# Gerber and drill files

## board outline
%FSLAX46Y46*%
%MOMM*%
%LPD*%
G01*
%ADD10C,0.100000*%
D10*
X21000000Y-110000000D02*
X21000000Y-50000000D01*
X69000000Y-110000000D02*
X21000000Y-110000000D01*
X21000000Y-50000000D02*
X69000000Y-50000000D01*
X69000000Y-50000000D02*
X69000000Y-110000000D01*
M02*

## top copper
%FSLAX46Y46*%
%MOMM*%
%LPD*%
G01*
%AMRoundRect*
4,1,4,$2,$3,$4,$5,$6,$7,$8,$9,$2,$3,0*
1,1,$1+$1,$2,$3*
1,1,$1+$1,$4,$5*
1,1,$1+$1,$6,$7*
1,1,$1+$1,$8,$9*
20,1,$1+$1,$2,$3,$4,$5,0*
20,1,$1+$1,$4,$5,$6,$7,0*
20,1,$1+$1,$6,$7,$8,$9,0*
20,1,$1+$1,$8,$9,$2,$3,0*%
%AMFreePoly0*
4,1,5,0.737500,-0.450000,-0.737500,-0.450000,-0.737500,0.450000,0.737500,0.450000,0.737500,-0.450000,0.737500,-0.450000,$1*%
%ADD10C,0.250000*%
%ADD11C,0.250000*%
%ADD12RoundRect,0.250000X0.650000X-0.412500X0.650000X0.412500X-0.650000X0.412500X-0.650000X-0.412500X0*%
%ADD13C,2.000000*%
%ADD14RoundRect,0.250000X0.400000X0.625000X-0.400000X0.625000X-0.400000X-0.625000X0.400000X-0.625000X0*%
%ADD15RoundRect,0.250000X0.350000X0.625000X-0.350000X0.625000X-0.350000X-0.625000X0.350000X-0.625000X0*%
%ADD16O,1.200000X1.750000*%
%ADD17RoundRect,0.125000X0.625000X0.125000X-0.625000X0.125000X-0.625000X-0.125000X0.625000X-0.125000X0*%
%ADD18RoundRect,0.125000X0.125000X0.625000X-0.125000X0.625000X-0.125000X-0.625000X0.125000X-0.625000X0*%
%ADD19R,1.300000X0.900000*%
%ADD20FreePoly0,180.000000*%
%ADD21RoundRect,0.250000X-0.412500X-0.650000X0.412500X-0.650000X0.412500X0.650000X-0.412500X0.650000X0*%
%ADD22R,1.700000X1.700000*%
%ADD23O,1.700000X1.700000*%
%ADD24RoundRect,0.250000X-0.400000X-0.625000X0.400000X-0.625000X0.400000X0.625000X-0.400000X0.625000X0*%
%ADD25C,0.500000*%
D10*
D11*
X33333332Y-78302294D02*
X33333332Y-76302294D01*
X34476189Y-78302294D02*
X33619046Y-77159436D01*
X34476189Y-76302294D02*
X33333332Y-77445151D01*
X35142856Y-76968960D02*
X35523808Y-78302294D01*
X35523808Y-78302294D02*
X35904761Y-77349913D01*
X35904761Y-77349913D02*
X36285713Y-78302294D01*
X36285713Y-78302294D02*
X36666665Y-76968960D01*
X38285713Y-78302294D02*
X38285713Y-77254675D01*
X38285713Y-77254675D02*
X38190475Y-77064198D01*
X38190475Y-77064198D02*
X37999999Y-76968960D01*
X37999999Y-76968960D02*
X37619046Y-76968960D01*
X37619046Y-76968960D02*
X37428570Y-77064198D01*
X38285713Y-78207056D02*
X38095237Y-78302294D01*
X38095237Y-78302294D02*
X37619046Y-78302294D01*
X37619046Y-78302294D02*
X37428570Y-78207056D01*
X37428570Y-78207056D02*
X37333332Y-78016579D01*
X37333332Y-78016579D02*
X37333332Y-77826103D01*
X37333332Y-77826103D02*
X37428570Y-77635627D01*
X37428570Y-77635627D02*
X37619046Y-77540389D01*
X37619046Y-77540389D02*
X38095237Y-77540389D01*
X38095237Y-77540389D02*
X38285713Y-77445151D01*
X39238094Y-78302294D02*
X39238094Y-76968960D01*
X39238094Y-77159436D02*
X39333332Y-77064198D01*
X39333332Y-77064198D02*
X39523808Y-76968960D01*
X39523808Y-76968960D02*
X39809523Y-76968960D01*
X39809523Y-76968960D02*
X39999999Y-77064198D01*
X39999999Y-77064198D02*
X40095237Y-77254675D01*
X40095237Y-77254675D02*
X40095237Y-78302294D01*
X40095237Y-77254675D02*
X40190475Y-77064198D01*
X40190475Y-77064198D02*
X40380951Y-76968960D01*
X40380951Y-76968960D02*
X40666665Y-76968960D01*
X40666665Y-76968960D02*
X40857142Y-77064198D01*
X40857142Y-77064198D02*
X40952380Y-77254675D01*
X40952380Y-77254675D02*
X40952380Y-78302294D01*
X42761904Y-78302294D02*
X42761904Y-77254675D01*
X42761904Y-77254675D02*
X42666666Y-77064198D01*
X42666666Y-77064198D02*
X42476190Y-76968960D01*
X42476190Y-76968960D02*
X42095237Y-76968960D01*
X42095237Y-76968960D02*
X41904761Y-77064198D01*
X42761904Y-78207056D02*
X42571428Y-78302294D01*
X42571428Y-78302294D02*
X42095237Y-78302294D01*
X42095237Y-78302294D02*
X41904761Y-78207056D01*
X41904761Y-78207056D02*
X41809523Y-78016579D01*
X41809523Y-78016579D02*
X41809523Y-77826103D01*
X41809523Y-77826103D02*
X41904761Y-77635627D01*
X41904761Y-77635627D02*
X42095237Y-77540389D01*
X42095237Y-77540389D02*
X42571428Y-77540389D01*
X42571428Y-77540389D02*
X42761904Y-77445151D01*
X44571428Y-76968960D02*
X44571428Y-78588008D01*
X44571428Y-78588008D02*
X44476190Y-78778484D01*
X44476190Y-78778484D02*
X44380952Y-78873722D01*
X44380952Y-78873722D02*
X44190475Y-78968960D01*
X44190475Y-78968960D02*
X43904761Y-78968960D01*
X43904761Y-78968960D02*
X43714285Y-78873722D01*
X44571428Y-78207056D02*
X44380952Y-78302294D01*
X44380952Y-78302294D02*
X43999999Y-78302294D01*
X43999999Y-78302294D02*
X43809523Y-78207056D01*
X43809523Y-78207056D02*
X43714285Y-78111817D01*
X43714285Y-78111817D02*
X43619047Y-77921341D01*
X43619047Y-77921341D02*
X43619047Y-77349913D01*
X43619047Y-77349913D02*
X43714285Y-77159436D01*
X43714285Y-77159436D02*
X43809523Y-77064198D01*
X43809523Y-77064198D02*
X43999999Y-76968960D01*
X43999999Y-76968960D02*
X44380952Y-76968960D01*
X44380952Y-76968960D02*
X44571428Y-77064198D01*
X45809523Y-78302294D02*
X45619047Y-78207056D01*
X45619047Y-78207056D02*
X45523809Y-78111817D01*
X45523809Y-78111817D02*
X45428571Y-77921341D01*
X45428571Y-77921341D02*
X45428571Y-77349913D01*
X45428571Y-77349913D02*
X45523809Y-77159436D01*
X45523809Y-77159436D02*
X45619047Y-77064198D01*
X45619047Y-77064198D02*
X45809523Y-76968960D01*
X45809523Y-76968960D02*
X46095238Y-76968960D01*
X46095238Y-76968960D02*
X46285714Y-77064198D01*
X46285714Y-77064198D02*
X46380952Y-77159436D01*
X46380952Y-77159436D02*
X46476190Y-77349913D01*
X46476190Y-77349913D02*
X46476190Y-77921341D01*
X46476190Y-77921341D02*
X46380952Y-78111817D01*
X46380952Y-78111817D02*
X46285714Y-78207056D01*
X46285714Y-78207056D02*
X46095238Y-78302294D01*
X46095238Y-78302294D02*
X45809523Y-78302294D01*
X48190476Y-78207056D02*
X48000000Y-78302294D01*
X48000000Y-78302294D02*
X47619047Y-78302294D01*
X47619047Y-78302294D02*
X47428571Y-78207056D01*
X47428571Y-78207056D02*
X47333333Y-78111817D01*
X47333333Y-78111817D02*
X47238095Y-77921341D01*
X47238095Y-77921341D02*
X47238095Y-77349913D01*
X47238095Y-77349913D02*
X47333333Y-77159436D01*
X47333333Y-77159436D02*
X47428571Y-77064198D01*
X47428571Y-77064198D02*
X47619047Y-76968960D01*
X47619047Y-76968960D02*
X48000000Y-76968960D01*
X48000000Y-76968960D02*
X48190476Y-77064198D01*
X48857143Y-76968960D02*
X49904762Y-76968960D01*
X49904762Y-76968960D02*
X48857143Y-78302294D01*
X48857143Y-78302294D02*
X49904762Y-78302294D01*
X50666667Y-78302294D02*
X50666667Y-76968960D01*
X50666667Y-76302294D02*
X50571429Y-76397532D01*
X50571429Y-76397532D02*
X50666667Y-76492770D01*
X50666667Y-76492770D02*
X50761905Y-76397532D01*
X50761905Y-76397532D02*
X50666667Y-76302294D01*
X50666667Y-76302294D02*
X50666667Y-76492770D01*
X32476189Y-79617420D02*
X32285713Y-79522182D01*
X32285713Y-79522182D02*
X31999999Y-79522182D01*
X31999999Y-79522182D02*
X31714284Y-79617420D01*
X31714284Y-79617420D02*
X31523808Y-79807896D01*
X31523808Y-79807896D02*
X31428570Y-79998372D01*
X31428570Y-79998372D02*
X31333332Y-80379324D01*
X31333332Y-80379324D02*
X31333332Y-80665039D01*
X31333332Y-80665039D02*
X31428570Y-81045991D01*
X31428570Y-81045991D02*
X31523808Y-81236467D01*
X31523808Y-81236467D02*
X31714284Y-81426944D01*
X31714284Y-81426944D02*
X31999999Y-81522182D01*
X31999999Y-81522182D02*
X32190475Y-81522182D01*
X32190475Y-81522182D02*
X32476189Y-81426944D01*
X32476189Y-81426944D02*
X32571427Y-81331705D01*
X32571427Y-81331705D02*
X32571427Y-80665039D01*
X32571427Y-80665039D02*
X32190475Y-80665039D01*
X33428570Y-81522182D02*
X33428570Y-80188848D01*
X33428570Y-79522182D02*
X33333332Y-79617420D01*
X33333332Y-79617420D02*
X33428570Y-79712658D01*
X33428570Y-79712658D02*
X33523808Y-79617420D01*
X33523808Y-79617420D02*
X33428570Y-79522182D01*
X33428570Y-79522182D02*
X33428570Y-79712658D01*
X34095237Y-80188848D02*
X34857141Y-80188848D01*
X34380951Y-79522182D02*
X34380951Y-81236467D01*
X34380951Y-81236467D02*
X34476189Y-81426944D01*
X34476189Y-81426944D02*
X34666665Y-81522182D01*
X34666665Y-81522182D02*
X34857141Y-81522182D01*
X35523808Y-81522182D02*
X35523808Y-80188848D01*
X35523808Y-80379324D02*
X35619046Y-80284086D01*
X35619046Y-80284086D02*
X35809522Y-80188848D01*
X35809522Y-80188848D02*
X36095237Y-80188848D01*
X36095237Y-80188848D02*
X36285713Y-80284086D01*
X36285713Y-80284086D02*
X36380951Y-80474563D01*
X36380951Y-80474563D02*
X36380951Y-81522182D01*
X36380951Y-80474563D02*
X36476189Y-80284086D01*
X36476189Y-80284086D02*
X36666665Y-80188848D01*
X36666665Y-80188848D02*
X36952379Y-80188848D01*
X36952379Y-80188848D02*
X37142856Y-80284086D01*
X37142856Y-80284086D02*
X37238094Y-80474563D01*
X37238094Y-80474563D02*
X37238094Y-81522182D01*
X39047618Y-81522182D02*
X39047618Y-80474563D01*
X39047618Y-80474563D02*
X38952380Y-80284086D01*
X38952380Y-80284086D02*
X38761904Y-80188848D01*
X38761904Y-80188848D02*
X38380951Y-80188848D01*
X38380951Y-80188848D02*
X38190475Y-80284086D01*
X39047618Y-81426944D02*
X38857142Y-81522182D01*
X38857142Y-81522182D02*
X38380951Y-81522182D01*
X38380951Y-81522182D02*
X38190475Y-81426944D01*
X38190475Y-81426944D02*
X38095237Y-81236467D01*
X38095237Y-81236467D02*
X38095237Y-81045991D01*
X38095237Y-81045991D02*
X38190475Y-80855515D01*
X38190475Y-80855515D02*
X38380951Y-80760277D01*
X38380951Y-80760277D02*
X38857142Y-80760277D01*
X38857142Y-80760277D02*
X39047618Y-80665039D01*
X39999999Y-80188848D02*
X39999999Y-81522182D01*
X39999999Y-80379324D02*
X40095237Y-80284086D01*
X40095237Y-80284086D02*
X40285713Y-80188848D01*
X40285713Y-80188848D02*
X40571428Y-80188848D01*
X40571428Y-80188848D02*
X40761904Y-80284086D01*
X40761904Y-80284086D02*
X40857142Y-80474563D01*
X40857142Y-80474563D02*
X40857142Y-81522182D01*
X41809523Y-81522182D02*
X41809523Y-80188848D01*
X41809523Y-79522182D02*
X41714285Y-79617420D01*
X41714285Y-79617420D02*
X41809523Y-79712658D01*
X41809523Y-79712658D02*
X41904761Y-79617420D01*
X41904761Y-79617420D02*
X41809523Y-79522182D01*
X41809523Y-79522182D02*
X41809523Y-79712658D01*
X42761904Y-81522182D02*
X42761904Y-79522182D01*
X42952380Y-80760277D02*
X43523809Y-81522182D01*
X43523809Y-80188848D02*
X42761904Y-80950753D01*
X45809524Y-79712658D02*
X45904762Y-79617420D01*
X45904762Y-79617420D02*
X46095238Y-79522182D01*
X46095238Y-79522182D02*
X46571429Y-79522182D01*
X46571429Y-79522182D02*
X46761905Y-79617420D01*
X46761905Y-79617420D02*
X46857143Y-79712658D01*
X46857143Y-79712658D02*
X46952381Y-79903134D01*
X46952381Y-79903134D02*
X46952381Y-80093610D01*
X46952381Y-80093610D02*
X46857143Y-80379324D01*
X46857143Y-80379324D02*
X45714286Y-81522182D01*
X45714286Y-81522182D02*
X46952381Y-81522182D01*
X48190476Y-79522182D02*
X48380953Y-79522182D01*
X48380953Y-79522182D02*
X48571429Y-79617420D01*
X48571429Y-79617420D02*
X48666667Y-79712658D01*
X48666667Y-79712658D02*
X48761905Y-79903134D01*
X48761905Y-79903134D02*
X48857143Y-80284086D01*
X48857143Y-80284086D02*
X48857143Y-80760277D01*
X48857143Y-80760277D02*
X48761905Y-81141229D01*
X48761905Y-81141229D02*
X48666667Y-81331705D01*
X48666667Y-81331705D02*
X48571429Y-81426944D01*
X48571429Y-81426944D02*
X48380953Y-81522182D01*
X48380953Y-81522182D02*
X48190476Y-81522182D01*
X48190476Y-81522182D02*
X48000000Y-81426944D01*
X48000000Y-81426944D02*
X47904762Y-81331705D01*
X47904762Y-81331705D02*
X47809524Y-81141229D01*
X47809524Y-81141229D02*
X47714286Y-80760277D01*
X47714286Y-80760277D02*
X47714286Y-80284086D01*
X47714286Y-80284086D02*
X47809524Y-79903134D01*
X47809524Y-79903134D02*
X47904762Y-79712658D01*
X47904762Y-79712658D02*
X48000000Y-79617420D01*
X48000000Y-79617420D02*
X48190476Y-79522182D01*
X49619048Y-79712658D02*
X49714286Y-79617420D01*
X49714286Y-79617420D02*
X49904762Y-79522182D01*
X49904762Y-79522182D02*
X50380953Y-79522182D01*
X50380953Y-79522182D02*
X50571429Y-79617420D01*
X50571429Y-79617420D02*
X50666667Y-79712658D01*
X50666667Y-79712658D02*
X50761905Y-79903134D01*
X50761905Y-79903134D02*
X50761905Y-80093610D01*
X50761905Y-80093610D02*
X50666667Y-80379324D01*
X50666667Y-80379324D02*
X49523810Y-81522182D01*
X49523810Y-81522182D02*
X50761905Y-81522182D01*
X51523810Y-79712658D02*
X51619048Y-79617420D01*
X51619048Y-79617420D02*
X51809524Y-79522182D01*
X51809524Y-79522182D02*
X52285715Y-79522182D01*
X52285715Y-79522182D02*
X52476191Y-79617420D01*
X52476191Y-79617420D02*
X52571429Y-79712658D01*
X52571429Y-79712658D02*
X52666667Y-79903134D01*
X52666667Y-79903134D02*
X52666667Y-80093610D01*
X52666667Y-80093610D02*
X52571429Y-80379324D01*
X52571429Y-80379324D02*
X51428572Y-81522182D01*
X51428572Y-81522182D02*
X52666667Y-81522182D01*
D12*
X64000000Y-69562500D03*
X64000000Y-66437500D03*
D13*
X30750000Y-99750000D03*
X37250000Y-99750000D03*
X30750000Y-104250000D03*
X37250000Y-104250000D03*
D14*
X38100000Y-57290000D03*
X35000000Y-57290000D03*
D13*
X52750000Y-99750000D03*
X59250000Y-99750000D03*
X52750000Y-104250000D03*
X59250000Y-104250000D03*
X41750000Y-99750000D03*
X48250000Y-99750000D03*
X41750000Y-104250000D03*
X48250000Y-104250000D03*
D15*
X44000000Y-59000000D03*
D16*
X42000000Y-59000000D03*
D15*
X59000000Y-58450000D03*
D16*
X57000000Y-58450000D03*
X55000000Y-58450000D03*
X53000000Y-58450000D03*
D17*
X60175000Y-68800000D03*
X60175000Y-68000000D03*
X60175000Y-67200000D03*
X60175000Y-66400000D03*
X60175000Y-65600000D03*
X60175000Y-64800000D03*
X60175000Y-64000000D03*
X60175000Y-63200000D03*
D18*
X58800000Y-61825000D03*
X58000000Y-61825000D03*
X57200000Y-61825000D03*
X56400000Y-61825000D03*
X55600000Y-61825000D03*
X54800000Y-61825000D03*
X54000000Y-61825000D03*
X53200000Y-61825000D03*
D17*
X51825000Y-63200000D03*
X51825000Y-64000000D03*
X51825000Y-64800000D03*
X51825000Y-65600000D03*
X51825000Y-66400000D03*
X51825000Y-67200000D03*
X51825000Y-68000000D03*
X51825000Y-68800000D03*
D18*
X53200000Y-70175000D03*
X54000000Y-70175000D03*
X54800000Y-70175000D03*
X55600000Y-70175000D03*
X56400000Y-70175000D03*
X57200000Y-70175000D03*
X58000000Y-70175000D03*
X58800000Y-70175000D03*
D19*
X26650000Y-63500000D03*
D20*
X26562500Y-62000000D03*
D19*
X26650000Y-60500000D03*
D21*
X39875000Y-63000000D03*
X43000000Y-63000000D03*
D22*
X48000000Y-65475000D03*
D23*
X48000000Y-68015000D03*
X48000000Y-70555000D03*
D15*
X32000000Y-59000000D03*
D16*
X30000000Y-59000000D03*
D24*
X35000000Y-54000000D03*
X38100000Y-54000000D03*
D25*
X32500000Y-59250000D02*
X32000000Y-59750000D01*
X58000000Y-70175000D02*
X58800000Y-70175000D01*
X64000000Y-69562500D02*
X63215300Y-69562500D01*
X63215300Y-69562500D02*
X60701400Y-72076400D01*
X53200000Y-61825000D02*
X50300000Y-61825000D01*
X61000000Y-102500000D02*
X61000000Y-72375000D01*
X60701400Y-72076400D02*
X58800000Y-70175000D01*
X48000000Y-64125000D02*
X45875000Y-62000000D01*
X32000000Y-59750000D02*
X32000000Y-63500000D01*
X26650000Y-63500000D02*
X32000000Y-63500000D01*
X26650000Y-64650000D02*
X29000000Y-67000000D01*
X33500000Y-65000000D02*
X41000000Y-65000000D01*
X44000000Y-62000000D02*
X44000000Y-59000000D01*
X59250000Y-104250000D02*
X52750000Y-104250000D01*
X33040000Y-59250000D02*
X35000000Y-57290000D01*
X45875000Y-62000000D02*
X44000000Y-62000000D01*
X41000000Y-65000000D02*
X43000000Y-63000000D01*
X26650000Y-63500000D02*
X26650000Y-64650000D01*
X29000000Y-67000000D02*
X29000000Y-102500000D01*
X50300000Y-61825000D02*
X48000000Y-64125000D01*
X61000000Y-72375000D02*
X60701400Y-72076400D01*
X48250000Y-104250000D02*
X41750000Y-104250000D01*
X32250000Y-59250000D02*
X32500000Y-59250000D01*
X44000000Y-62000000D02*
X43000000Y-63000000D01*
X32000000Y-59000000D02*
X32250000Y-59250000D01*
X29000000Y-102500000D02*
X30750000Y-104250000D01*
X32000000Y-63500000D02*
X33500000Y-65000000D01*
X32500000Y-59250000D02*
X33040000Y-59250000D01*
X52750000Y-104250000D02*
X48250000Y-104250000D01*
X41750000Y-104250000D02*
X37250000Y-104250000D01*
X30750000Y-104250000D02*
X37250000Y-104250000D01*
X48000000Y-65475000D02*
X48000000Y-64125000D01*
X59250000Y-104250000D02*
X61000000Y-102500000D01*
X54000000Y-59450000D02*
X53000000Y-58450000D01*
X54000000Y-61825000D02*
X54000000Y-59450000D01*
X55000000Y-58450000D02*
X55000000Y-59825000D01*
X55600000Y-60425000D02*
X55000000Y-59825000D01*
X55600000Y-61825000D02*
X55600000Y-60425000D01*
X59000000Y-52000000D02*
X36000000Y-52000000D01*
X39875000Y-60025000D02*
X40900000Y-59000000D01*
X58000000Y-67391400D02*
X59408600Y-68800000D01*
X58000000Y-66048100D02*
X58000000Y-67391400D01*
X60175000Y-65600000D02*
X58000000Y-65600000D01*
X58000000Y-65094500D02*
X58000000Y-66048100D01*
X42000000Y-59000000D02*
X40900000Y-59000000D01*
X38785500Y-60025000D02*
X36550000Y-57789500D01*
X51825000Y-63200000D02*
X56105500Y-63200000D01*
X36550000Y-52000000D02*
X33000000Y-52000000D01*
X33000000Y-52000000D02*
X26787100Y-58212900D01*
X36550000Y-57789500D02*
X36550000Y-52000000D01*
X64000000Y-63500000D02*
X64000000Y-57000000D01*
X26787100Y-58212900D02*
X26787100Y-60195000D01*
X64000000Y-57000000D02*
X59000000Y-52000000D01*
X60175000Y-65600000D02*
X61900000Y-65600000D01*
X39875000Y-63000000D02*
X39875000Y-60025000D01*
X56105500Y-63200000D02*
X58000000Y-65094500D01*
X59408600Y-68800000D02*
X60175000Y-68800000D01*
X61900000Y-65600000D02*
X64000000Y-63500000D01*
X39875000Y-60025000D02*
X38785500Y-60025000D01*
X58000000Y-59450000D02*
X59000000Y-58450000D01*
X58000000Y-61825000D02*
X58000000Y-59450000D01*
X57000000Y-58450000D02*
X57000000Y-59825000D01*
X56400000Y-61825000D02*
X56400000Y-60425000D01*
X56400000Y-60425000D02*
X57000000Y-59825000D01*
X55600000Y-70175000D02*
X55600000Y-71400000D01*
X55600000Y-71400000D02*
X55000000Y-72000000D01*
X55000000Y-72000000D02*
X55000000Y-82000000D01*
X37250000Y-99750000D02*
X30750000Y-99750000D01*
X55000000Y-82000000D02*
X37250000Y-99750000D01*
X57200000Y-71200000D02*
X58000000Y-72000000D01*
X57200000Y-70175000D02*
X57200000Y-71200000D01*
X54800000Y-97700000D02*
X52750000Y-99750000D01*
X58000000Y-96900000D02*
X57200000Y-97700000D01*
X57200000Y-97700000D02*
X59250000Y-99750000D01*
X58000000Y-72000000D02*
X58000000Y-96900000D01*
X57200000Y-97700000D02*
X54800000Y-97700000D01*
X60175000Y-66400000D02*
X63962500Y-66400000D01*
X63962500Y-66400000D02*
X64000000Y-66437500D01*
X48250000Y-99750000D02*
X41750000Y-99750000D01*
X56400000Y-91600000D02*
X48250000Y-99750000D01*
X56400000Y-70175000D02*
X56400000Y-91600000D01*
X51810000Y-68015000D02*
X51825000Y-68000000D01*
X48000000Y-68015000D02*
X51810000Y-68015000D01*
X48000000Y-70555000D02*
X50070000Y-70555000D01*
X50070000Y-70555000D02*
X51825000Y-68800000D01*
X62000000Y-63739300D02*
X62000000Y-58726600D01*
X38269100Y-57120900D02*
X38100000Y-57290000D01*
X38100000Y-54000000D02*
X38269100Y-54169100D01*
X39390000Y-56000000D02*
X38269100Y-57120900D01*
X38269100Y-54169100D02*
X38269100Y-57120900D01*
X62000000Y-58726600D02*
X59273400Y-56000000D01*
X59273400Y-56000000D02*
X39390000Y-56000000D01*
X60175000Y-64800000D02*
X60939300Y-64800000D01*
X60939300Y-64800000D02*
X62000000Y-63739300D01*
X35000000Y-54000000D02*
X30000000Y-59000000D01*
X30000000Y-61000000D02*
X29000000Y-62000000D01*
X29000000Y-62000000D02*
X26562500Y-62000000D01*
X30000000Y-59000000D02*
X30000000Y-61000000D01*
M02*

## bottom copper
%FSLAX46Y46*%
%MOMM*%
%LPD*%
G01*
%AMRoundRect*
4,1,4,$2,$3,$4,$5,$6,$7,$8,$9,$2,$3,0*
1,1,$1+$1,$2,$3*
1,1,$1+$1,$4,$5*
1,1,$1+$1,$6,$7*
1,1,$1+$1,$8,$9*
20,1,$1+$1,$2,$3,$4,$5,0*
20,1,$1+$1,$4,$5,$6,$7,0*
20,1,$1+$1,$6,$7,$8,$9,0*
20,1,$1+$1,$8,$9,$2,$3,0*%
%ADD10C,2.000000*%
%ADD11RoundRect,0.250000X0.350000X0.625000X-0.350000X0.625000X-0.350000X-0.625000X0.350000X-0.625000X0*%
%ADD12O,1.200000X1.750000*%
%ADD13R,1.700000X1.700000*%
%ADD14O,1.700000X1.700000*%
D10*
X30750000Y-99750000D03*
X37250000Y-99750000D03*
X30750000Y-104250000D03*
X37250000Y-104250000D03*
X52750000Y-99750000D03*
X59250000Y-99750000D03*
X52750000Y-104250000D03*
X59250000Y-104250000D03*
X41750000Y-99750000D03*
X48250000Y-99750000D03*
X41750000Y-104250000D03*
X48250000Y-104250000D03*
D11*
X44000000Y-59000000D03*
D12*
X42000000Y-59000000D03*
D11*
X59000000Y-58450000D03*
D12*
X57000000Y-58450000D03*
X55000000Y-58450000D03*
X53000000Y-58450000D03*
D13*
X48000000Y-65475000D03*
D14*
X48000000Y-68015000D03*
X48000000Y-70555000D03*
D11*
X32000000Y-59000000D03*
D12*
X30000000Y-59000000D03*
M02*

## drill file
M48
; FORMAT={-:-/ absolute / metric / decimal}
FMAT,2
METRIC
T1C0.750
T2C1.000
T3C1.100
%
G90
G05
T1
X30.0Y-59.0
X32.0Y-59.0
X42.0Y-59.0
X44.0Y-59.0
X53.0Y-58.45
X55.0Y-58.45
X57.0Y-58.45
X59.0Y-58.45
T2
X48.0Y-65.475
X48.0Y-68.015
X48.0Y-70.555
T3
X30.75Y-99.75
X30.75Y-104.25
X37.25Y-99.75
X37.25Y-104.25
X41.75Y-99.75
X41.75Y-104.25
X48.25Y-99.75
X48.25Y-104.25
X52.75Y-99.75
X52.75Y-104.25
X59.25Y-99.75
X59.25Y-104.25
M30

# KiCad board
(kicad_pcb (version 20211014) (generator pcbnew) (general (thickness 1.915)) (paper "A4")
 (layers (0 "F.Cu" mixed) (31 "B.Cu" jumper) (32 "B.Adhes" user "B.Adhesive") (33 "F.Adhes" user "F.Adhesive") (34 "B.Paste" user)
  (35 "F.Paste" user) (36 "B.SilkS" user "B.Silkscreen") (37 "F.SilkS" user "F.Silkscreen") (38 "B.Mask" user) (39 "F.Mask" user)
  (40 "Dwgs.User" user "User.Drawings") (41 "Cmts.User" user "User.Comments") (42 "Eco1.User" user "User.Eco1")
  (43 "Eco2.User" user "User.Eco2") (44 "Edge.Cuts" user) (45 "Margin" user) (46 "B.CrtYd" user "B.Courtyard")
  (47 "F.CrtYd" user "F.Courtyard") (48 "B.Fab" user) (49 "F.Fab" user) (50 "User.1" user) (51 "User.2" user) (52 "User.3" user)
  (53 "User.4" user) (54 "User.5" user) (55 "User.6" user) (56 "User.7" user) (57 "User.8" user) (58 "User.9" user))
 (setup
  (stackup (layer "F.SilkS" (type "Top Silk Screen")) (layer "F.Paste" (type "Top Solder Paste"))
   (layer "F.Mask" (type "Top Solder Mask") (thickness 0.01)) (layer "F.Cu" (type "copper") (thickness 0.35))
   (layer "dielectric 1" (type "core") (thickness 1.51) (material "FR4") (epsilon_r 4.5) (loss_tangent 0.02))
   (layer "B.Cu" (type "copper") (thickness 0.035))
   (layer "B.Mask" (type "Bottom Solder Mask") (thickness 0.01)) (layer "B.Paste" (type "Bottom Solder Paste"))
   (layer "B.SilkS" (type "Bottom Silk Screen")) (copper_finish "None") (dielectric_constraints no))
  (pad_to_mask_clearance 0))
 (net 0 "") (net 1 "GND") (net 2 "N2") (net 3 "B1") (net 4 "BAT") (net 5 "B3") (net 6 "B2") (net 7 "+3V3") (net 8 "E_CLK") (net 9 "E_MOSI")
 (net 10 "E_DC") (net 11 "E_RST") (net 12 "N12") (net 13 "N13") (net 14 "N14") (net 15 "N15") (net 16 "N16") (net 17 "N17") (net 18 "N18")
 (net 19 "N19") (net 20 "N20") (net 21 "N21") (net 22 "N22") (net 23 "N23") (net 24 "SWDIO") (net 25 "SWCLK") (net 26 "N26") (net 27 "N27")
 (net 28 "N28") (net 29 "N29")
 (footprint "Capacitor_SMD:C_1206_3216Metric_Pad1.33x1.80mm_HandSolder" (layer "F.Cu") (at 64 68 90)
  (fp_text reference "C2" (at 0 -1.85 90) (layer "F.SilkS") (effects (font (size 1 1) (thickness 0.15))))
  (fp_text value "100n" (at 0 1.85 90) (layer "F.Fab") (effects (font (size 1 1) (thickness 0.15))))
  (pad "1" smd roundrect (at -1.5625 0 90) (size 1.325 1.8) (layers "F.Cu" "F.Paste" "F.Mask") (roundrect_rratio 0.188679) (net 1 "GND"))
  (pad "2" smd roundrect (at 1.5625 0 90) (size 1.325 1.8) (layers "F.Cu" "F.Paste" "F.Mask") (roundrect_rratio 0.188679) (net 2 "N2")))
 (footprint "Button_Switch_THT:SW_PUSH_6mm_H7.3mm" (layer "F.Cu") (at 30.75 99.75)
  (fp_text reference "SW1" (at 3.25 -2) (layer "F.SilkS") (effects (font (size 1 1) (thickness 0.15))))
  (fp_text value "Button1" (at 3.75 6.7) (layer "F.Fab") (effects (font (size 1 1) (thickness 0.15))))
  (pad "1" thru_hole circle (at 0 0 90) (size 2 2) (drill 1.1) (layers *.Cu *.Mask) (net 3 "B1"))
  (pad "1" thru_hole circle (at 6.5 0 90) (size 2 2) (drill 1.1) (layers *.Cu *.Mask) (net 3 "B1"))
  (pad "2" thru_hole circle (at 0 4.5 90) (size 2 2) (drill 1.1) (layers *.Cu *.Mask) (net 1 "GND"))
  (pad "2" thru_hole circle (at 6.5 4.5 90) (size 2 2) (drill 1.1) (layers *.Cu *.Mask) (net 1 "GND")))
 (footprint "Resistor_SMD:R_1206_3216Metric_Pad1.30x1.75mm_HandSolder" (layer "F.Cu") (at 36.55 57.29 180)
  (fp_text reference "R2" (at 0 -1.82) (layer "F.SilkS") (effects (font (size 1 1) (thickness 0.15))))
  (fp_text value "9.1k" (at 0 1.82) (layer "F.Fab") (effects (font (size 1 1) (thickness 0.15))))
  (pad "1" smd roundrect (at -1.55 0 180) (size 1.3 1.75) (layers "F.Cu" "F.Paste" "F.Mask") (roundrect_rratio 0.192308) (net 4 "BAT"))
  (pad "2" smd roundrect (at 1.55 0 180) (size 1.3 1.75) (layers "F.Cu" "F.Paste" "F.Mask") (roundrect_rratio 0.192308) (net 1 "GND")))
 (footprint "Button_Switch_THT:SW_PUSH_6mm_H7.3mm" (layer "F.Cu") (at 52.75 99.75)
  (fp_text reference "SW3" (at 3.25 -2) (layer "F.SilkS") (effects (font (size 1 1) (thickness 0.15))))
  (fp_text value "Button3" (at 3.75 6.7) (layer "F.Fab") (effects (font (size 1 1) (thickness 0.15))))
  (pad "1" thru_hole circle (at 0 0 90) (size 2 2) (drill 1.1) (layers *.Cu *.Mask) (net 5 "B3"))
  (pad "1" thru_hole circle (at 6.5 0 90) (size 2 2) (drill 1.1) (layers *.Cu *.Mask) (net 5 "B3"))
  (pad "2" thru_hole circle (at 0 4.5 90) (size 2 2) (drill 1.1) (layers *.Cu *.Mask) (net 1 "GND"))
  (pad "2" thru_hole circle (at 6.5 4.5 90) (size 2 2) (drill 1.1) (layers *.Cu *.Mask) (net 1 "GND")))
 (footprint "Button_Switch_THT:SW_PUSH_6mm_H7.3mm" (layer "F.Cu") (at 41.75 99.75)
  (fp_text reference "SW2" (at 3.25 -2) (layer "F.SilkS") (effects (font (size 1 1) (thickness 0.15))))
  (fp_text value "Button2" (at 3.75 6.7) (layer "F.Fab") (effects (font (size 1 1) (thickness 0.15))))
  (pad "1" thru_hole circle (at 0 0 90) (size 2 2) (drill 1.1) (layers *.Cu *.Mask) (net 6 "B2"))
  (pad "1" thru_hole circle (at 6.5 0 90) (size 2 2) (drill 1.1) (layers *.Cu *.Mask) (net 6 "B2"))
  (pad "2" thru_hole circle (at 0 4.5 90) (size 2 2) (drill 1.1) (layers *.Cu *.Mask) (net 1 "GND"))
  (pad "2" thru_hole circle (at 6.5 4.5 90) (size 2 2) (drill 1.1) (layers *.Cu *.Mask) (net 1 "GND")))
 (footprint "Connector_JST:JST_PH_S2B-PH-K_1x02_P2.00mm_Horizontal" (layer "F.Cu") (at 44 59 180)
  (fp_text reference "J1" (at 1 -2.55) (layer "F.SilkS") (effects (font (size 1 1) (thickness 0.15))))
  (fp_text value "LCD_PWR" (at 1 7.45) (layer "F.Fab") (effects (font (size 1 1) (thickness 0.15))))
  (pad "1" thru_hole roundrect (at 0 0 180) (size 1.2 1.75) (drill 0.75) (layers *.Cu *.Mask) (roundrect_rratio 0.208333) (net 1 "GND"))
  (pad "2" thru_hole oval (at 2 0 180) (size 1.2 1.75) (drill 0.75) (layers *.Cu *.Mask) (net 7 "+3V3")))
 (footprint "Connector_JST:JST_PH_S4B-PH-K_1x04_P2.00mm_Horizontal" (layer "F.Cu") (at 59 58.45 180)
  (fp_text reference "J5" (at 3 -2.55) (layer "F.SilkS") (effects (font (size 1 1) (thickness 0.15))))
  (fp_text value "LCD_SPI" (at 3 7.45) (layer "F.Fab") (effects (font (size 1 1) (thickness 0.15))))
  (pad "1" thru_hole roundrect (at 0 0 180) (size 1.2 1.75) (drill 0.75) (layers *.Cu *.Mask) (roundrect_rratio 0.208333) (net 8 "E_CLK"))
  (pad "2" thru_hole oval (at 2 0 180) (size 1.2 1.75) (drill 0.75) (layers *.Cu *.Mask) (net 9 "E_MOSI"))
  (pad "3" thru_hole oval (at 4 0 180) (size 1.2 1.75) (drill 0.75) (layers *.Cu *.Mask) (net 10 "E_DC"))
  (pad "4" thru_hole oval (at 6 0 180) (size 1.2 1.75) (drill 0.75) (layers *.Cu *.Mask) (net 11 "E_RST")))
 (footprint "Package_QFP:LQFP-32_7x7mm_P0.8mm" (layer "F.Cu") (at 56 66 180)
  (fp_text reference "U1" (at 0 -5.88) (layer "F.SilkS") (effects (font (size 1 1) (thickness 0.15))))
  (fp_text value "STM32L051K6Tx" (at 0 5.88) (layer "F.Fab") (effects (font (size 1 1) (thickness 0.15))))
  (pad "1" smd roundrect (at -4.175 -2.8 180) (size 1.5 0.5) (layers "F.Cu" "F.Paste" "F.Mask") (roundrect_rratio 0.25) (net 7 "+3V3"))
  (pad "2" smd roundrect (at -4.175 -2 180) (size 1.5 0.5) (layers "F.Cu" "F.Paste" "F.Mask") (roundrect_rratio 0.25) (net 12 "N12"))
  (pad "3" smd roundrect (at -4.175 -1.2 180) (size 1.5 0.5) (layers "F.Cu" "F.Paste" "F.Mask") (roundrect_rratio 0.25) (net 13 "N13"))
  (pad "4" smd roundrect (at -4.175 -0.4 180) (size 1.5 0.5) (layers "F.Cu" "F.Paste" "F.Mask") (roundrect_rratio 0.25) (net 2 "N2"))
  (pad "5" smd roundrect (at -4.175 0.4 180) (size 1.5 0.5) (layers "F.Cu" "F.Paste" "F.Mask") (roundrect_rratio 0.25) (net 7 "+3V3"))
  (pad "6" smd roundrect (at -4.175 1.2 180) (size 1.5 0.5) (layers "F.Cu" "F.Paste" "F.Mask") (roundrect_rratio 0.25) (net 4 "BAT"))
  (pad "7" smd roundrect (at -4.175 2 180) (size 1.5 0.5) (layers "F.Cu" "F.Paste" "F.Mask") (roundrect_rratio 0.25) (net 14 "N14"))
  (pad "8" smd roundrect (at -4.175 2.8 180) (size 1.5 0.5) (layers "F.Cu" "F.Paste" "F.Mask") (roundrect_rratio 0.25) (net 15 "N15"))
  (pad "9" smd roundrect (at -2.8 4.175 180) (size 0.5 1.5) (layers "F.Cu" "F.Paste" "F.Mask") (roundrect_rratio 0.25) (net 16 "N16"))
  (pad "10" smd roundrect (at -2 4.175 180) (size 0.5 1.5) (layers "F.Cu" "F.Paste" "F.Mask") (roundrect_rratio 0.25) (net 8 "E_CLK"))
  (pad "11" smd roundrect (at -1.2 4.175 180) (size 0.5 1.5) (layers "F.Cu" "F.Paste" "F.Mask") (roundrect_rratio 0.25) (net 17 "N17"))
  (pad "12" smd roundrect (at -0.4 4.175 180) (size 0.5 1.5) (layers "F.Cu" "F.Paste" "F.Mask") (roundrect_rratio 0.25) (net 9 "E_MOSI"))
  (pad "13" smd roundrect (at 0.4 4.175 180) (size 0.5 1.5) (layers "F.Cu" "F.Paste" "F.Mask") (roundrect_rratio 0.25) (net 10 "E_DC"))
  (pad "14" smd roundrect (at 1.2 4.175 180) (size 0.5 1.5) (layers "F.Cu" "F.Paste" "F.Mask") (roundrect_rratio 0.25) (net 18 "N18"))
  (pad "15" smd roundrect (at 2 4.175 180) (size 0.5 1.5) (layers "F.Cu" "F.Paste" "F.Mask") (roundrect_rratio 0.25) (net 11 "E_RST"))
  (pad "16" smd roundrect (at 2.8 4.175 180) (size 0.5 1.5) (layers "F.Cu" "F.Paste" "F.Mask") (roundrect_rratio 0.25) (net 1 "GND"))
  (pad "17" smd roundrect (at 4.175 2.8 180) (size 1.5 0.5) (layers "F.Cu" "F.Paste" "F.Mask") (roundrect_rratio 0.25) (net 7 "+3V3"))
  (pad "18" smd roundrect (at 4.175 2 180) (size 1.5 0.5) (layers "F.Cu" "F.Paste" "F.Mask") (roundrect_rratio 0.25) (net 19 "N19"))
  (pad "19" smd roundrect (at 4.175 1.2 180) (size 1.5 0.5) (layers "F.Cu" "F.Paste" "F.Mask") (roundrect_rratio 0.25) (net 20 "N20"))
  (pad "20" smd roundrect (at 4.175 0.4 180) (size 1.5 0.5) (layers "F.Cu" "F.Paste" "F.Mask") (roundrect_rratio 0.25) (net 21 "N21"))
  (pad "21" smd roundrect (at 4.175 -0.4 180) (size 1.5 0.5) (layers "F.Cu" "F.Paste" "F.Mask") (roundrect_rratio 0.25) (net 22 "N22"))
  (pad "22" smd roundrect (at 4.175 -1.2 180) (size 1.5 0.5) (layers "F.Cu" "F.Paste" "F.Mask") (roundrect_rratio 0.25) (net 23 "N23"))
  (pad "23" smd roundrect (at 4.175 -2 180) (size 1.5 0.5) (layers "F.Cu" "F.Paste" "F.Mask") (roundrect_rratio 0.25) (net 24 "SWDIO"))
  (pad "24" smd roundrect (at 4.175 -2.8 180) (size 1.5 0.5) (layers "F.Cu" "F.Paste" "F.Mask") (roundrect_rratio 0.25) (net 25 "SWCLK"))
  (pad "25" smd roundrect (at 2.8 -4.175 180) (size 0.5 1.5) (layers "F.Cu" "F.Paste" "F.Mask") (roundrect_rratio 0.25) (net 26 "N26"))
  (pad "26" smd roundrect (at 2 -4.175 180) (size 0.5 1.5) (layers "F.Cu" "F.Paste" "F.Mask") (roundrect_rratio 0.25) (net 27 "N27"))
  (pad "27" smd roundrect (at 1.2 -4.175 180) (size 0.5 1.5) (layers "F.Cu" "F.Paste" "F.Mask") (roundrect_rratio 0.25) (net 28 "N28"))
  (pad "28" smd roundrect (at 0.4 -4.175 180) (size 0.5 1.5) (layers "F.Cu" "F.Paste" "F.Mask") (roundrect_rratio 0.25) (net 3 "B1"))
  (pad "29" smd roundrect (at -0.4 -4.175 180) (size 0.5 1.5) (layers "F.Cu" "F.Paste" "F.Mask") (roundrect_rratio 0.25) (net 6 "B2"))
  (pad "30" smd roundrect (at -1.2 -4.175 180) (size 0.5 1.5) (layers "F.Cu" "F.Paste" "F.Mask") (roundrect_rratio 0.25) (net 5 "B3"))
  (pad "31" smd roundrect (at -2 -4.175 180) (size 0.5 1.5) (layers "F.Cu" "F.Paste" "F.Mask") (roundrect_rratio 0.25) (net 1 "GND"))
  (pad "32" smd roundrect (at -2.8 -4.175 180) (size 0.5 1.5) (layers "F.Cu" "F.Paste" "F.Mask") (roundrect_rratio 0.25) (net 1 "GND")))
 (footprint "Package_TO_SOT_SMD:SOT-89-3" (layer "F.Cu") (at 25 62 180)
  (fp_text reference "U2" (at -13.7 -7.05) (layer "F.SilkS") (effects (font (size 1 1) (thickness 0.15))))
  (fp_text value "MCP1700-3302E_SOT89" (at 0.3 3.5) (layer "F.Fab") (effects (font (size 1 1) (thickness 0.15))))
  (pad "1" smd rect (at -1.65 -1.5 180) (size 1.3 0.9) (layers "F.Cu" "F.Paste" "F.Mask") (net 1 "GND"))
  (pad "2" smd custom (at -1.5625 0 180) (size 1.475 0.9) (layers "F.Cu" "F.Paste" "F.Mask") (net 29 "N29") (zone_connect 2)
   (options (clearance outline) (anchor rect)) (primitives))
  (pad "3" smd rect (at -1.65 1.5 180) (size 1.3 0.9) (layers "F.Cu" "F.Paste" "F.Mask") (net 7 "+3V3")))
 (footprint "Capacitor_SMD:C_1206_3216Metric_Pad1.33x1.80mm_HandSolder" (layer "F.Cu") (at 41.4375 63)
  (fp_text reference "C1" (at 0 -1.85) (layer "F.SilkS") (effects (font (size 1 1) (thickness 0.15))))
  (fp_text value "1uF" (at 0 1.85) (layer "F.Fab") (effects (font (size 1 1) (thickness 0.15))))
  (pad "1" smd roundrect (at -1.5625 0) (size 1.325 1.8) (layers "F.Cu" "F.Paste" "F.Mask") (roundrect_rratio 0.188679) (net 7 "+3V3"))
  (pad "2" smd roundrect (at 1.5625 0) (size 1.325 1.8) (layers "F.Cu" "F.Paste" "F.Mask") (roundrect_rratio 0.188679) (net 1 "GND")))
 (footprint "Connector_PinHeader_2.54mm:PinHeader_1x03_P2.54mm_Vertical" (layer "F.Cu") (at 48 65.475)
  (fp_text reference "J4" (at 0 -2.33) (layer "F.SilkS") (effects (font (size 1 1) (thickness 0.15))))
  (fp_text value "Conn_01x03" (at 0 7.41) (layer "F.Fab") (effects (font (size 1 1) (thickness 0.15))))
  (pad "1" thru_hole rect (at 0 0) (size 1.7 1.7) (drill 1) (layers *.Cu *.Mask) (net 1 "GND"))
  (pad "2" thru_hole oval (at 0 2.54) (size 1.7 1.7) (drill 1) (layers *.Cu *.Mask) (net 24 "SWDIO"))
  (pad "3" thru_hole oval (at 0 5.08) (size 1.7 1.7) (drill 1) (layers *.Cu *.Mask) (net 25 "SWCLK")))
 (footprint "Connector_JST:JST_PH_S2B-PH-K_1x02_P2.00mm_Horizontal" (layer "F.Cu") (at 32 59 180)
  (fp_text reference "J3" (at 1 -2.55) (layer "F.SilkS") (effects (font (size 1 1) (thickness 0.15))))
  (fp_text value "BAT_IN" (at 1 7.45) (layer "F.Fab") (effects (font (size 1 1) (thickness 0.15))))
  (pad "1" thru_hole roundrect (at 0 0 180) (size 1.2 1.75) (drill 0.75) (layers *.Cu *.Mask) (roundrect_rratio 0.208333) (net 1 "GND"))
  (pad "2" thru_hole oval (at 2 0 180) (size 1.2 1.75) (drill 0.75) (layers *.Cu *.Mask) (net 29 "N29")))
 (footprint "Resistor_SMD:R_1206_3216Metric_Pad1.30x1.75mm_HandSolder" (layer "F.Cu") (at 36.55 54)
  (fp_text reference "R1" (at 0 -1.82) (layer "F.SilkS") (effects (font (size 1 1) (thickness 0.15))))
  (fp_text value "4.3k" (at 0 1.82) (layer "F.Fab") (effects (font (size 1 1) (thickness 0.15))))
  (pad "1" smd roundrect (at -1.55 0) (size 1.3 1.75) (layers "F.Cu" "F.Paste" "F.Mask") (roundrect_rratio 0.192308) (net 29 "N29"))
  (pad "2" smd roundrect (at 1.55 0) (size 1.3 1.75) (layers "F.Cu" "F.Paste" "F.Mask") (roundrect_rratio 0.192308) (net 4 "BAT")))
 (gr_line (start 21 110) (end 21 50) (layer "Edge.Cuts") (width 0.1))
 (gr_line (start 69 110) (end 21 110) (layer "Edge.Cuts") (width 0.1))
 (gr_line (start 21 50) (end 69 50) (layer "Edge.Cuts") (width 0.1))
 (gr_line (start 69 50) (end 69 110) (layer "Edge.Cuts") (width 0.1))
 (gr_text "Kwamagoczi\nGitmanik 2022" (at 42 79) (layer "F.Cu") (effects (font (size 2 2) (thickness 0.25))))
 (segment (start 32.5 59.25) (end 32 59.75) (width 0.5) (layer "F.Cu") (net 1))
 (segment (start 58 70.175) (end 58.8 70.175) (width 0.5) (layer "F.Cu") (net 1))
 (segment (start 64 69.5625) (end 63.2153 69.5625) (width 0.5) (layer "F.Cu") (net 1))
 (segment (start 63.2153 69.5625) (end 60.7014 72.0764) (width 0.5) (layer "F.Cu") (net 1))
 (segment (start 53.2 61.825) (end 50.3 61.825) (width 0.5) (layer "F.Cu") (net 1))
 (segment (start 61 102.5) (end 61 72.375) (width 0.5) (layer "F.Cu") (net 1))
 (segment (start 60.7014 72.0764) (end 58.8 70.175) (width 0.5) (layer "F.Cu") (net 1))
 (segment (start 48 64.125) (end 45.875 62) (width 0.5) (layer "F.Cu") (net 1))
 (segment (start 32 59.75) (end 32 63.5) (width 0.5) (layer "F.Cu") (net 1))
 (segment (start 26.65 63.5) (end 32 63.5) (width 0.5) (layer "F.Cu") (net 1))
 (segment (start 26.65 64.65) (end 29 67) (width 0.5) (layer "F.Cu") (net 1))
 (segment (start 33.5 65) (end 41 65) (width 0.5) (layer "F.Cu") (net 1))
 (segment (start 44 62) (end 44 59) (width 0.5) (layer "F.Cu") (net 1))
 (segment (start 59.25 104.25) (end 52.75 104.25) (width 0.5) (layer "F.Cu") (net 1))
 (segment (start 33.04 59.25) (end 35 57.29) (width 0.5) (layer "F.Cu") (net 1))
 (segment (start 45.875 62) (end 44 62) (width 0.5) (layer "F.Cu") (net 1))
 (segment (start 41 65) (end 43 63) (width 0.5) (layer "F.Cu") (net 1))
 (segment (start 26.65 63.5) (end 26.65 64.65) (width 0.5) (layer "F.Cu") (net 1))
 (segment (start 29 67) (end 29 102.5) (width 0.5) (layer "F.Cu") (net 1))
 (segment (start 50.3 61.825) (end 48 64.125) (width 0.5) (layer "F.Cu") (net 1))
 (segment (start 61 72.375) (end 60.7014 72.0764) (width 0.5) (layer "F.Cu") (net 1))
 (segment (start 48.25 104.25) (end 41.75 104.25) (width 0.5) (layer "F.Cu") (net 1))
 (segment (start 32.25 59.25) (end 32.5 59.25) (width 0.5) (layer "F.Cu") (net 1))
 (segment (start 44 62) (end 43 63) (width 0.5) (layer "F.Cu") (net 1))
 (segment (start 32 59) (end 32.25 59.25) (width 0.5) (layer "F.Cu") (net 1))
 (segment (start 29 102.5) (end 30.75 104.25) (width 0.5) (layer "F.Cu") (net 1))
 (segment (start 32 63.5) (end 33.5 65) (width 0.5) (layer "F.Cu") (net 1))
 (segment (start 32.5 59.25) (end 33.04 59.25) (width 0.5) (layer "F.Cu") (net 1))
 (segment (start 52.75 104.25) (end 48.25 104.25) (width 0.5) (layer "F.Cu") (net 1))
 (segment (start 41.75 104.25) (end 37.25 104.25) (width 0.5) (layer "F.Cu") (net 1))
 (segment (start 30.75 104.25) (end 37.25 104.25) (width 0.5) (layer "F.Cu") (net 1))
 (segment (start 48 65.475) (end 48 64.125) (width 0.5) (layer "F.Cu") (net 1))
 (segment (start 59.25 104.25) (end 61 102.5) (width 0.5) (layer "F.Cu") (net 1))
 (segment (start 54 59.45) (end 53 58.45) (width 0.5) (layer "F.Cu") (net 11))
 (segment (start 54 61.825) (end 54 59.45) (width 0.5) (layer "F.Cu") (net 11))
 (segment (start 55 58.45) (end 55 59.825) (width 0.5) (layer "F.Cu") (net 10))
 (segment (start 55.6 60.425) (end 55 59.825) (width 0.5) (layer "F.Cu") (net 10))
 (segment (start 55.6 61.825) (end 55.6 60.425) (width 0.5) (layer "F.Cu") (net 10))
 (segment (start 59 52) (end 36 52) (width 0.5) (layer "F.Cu") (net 7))
 (segment (start 39.875 60.025) (end 40.9 59) (width 0.5) (layer "F.Cu") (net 7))
 (segment (start 58 67.3914) (end 59.4086 68.8) (width 0.5) (layer "F.Cu") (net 7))
 (segment (start 58 66.0481) (end 58 67.3914) (width 0.5) (layer "F.Cu") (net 7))
 (segment (start 60.175 65.6) (end 58 65.6) (width 0.5) (layer "F.Cu") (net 7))
 (segment (start 58 65.0945) (end 58 66.0481) (width 0.5) (layer "F.Cu") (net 7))
 (segment (start 42 59) (end 40.9 59) (width 0.5) (layer "F.Cu") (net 7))
 (segment (start 38.7855 60.025) (end 36.55 57.7895) (width 0.5) (layer "F.Cu") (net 7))
 (segment (start 51.825 63.2) (end 56.1055 63.2) (width 0.5) (layer "F.Cu") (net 7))
 (segment (start 36.55 52) (end 33 52) (width 0.5) (layer "F.Cu") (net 7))
 (segment (start 33 52) (end 26.7871 58.2129) (width 0.5) (layer "F.Cu") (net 7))
 (segment (start 36.55 57.7895) (end 36.55 52) (width 0.5) (layer "F.Cu") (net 7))
 (segment (start 64 63.5) (end 64 57) (width 0.5) (layer "F.Cu") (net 7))
 (segment (start 26.7871 58.2129) (end 26.7871 60.195) (width 0.5) (layer "F.Cu") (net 7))
 (segment (start 64 57) (end 59 52) (width 0.5) (layer "F.Cu") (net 7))
 (segment (start 60.175 65.6) (end 61.9 65.6) (width 0.5) (layer "F.Cu") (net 7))
 (segment (start 39.875 63) (end 39.875 60.025) (width 0.5) (layer "F.Cu") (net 7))
 (segment (start 56.1055 63.2) (end 58 65.0945) (width 0.5) (layer "F.Cu") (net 7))
 (segment (start 59.4086 68.8) (end 60.175 68.8) (width 0.5) (layer "F.Cu") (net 7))
 (segment (start 61.9 65.6) (end 64 63.5) (width 0.5) (layer "F.Cu") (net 7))
 (segment (start 39.875 60.025) (end 38.7855 60.025) (width 0.5) (layer "F.Cu") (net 7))
 (segment (start 58 59.45) (end 59 58.45) (width 0.5) (layer "F.Cu") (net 8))
 (segment (start 58 61.825) (end 58 59.45) (width 0.5) (layer "F.Cu") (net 8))
 (segment (start 57 58.45) (end 57 59.825) (width 0.5) (layer "F.Cu") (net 9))
 (segment (start 56.4 61.825) (end 56.4 60.425) (width 0.5) (layer "F.Cu") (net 9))
 (segment (start 56.4 60.425) (end 57 59.825) (width 0.5) (layer "F.Cu") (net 9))
 (segment (start 55.6 70.175) (end 55.6 71.4) (width 0.5) (layer "F.Cu") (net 3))
 (segment (start 55.6 71.4) (end 55 72) (width 0.5) (layer "F.Cu") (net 3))
 (segment (start 55 72) (end 55 82) (width 0.5) (layer "F.Cu") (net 3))
 (segment (start 37.25 99.75) (end 30.75 99.75) (width 0.5) (layer "F.Cu") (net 3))
 (segment (start 55 82) (end 37.25 99.75) (width 0.5) (layer "F.Cu") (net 3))
 (segment (start 57.2 71.2) (end 58 72) (width 0.5) (layer "F.Cu") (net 5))
 (segment (start 57.2 70.175) (end 57.2 71.2) (width 0.5) (layer "F.Cu") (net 5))
 (segment (start 54.8 97.7) (end 52.75 99.75) (width 0.5) (layer "F.Cu") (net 5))
 (segment (start 58 96.9) (end 57.2 97.7) (width 0.5) (layer "F.Cu") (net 5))
 (segment (start 57.2 97.7) (end 59.25 99.75) (width 0.5) (layer "F.Cu") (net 5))
 (segment (start 58 72) (end 58 96.9) (width 0.5) (layer "F.Cu") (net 5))
 (segment (start 57.2 97.7) (end 54.8 97.7) (width 0.5) (layer "F.Cu") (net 5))
 (segment (start 60.175 66.4) (end 63.9625 66.4) (width 0.5) (layer "F.Cu") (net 2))
 (segment (start 63.9625 66.4) (end 64 66.4375) (width 0.5) (layer "F.Cu") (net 2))
 (segment (start 48.25 99.75) (end 41.75 99.75) (width 0.5) (layer "F.Cu") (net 6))
 (segment (start 56.4 91.6) (end 48.25 99.75) (width 0.5) (layer "F.Cu") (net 6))
 (segment (start 56.4 70.175) (end 56.4 91.6) (width 0.5) (layer "F.Cu") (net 6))
 (segment (start 51.81 68.015) (end 51.825 68) (width 0.5) (layer "F.Cu") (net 24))
 (segment (start 48 68.015) (end 51.81 68.015) (width 0.5) (layer "F.Cu") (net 24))
 (segment (start 48 70.555) (end 50.07 70.555) (width 0.5) (layer "F.Cu") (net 25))
 (segment (start 50.07 70.555) (end 51.825 68.8) (width 0.5) (layer "F.Cu") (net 25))
 (segment (start 62 63.7393) (end 62 58.7266) (width 0.5) (layer "F.Cu") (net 4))
 (segment (start 38.2691 57.1209) (end 38.1 57.29) (width 0.5) (layer "F.Cu") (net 4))
 (segment (start 38.1 54) (end 38.2691 54.1691) (width 0.5) (layer "F.Cu") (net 4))
 (segment (start 39.39 56) (end 38.2691 57.1209) (width 0.5) (layer "F.Cu") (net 4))
 (segment (start 38.2691 54.1691) (end 38.2691 57.1209) (width 0.5) (layer "F.Cu") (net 4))
 (segment (start 62 58.7266) (end 59.2734 56) (width 0.5) (layer "F.Cu") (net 4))
 (segment (start 59.2734 56) (end 39.39 56) (width 0.5) (layer "F.Cu") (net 4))
 (segment (start 60.175 64.8) (end 60.9393 64.8) (width 0.5) (layer "F.Cu") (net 4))
 (segment (start 60.9393 64.8) (end 62 63.7393) (width 0.5) (layer "F.Cu") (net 4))
 (segment (start 35 54) (end 30 59) (width 0.5) (layer "F.Cu") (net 29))
 (segment (start 30 61) (end 29 62) (width 0.5) (layer "F.Cu") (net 29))
 (segment (start 29 62) (end 26.5625 62) (width 0.5) (layer "F.Cu") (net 29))
 (segment (start 30 59) (end 30 61) (width 0.5) (layer "F.Cu") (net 29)))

